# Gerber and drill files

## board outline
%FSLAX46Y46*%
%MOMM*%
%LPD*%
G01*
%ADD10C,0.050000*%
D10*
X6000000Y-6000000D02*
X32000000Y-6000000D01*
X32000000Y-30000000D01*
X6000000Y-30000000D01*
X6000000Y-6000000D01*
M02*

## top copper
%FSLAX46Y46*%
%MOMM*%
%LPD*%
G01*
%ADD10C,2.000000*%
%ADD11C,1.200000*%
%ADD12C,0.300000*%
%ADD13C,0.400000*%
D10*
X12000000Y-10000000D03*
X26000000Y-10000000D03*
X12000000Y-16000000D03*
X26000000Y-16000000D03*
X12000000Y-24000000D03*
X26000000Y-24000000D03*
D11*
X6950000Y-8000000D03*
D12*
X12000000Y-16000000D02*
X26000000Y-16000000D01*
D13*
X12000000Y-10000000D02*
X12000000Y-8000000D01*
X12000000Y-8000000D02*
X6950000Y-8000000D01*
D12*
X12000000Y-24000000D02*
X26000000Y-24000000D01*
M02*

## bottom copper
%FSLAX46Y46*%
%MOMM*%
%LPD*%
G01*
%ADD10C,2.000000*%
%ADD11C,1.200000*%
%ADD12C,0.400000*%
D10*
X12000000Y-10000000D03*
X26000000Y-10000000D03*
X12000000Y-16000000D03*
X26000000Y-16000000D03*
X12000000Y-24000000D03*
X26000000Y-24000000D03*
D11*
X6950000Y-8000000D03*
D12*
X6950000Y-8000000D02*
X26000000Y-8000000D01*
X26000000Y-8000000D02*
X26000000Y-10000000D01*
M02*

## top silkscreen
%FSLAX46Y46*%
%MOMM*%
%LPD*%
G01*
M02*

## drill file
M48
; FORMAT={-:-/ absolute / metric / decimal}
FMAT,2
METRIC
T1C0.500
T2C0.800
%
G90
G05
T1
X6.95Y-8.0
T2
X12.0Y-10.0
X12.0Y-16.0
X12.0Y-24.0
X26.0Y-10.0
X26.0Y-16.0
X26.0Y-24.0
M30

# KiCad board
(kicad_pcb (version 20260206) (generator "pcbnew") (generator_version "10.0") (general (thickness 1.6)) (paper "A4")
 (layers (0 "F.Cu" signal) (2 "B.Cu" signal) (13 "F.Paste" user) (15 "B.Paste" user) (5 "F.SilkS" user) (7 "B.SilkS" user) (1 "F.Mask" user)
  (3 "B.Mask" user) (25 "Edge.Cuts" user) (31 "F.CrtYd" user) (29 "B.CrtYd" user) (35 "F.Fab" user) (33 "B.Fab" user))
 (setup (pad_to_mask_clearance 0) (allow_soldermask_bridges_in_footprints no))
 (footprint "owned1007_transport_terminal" (layer "F.Cu") (at 12 10)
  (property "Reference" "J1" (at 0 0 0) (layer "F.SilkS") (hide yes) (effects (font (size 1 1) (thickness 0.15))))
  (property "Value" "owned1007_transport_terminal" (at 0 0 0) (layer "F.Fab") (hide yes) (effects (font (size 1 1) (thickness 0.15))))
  (pad "1" thru_hole circle (at 0 0) (size 2 2) (drill 0.8) (layers "*.Cu" "*.Mask") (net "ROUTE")))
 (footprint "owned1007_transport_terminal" (layer "F.Cu") (at 26 10)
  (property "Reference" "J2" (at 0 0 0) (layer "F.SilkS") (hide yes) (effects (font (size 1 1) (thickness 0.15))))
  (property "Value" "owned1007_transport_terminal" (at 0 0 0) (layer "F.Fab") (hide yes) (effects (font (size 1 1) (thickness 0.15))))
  (pad "1" thru_hole circle (at 0 0) (size 2 2) (drill 0.8) (layers "*.Cu" "*.Mask") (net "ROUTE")))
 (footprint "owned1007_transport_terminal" (layer "F.Cu") (at 12 16)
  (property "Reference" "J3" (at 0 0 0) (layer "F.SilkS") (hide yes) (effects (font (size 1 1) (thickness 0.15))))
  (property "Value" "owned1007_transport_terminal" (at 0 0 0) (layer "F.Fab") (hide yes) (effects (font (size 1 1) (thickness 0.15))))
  (pad "1" thru_hole circle (at 0 0) (size 2 2) (drill 0.8) (layers "*.Cu" "*.Mask") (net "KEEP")))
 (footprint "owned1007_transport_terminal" (layer "F.Cu") (at 26 16)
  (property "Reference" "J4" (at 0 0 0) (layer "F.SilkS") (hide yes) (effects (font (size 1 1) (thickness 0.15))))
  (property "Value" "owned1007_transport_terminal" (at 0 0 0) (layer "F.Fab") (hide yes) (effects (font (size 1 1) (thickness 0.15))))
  (pad "1" thru_hole circle (at 0 0) (size 2 2) (drill 0.8) (layers "*.Cu" "*.Mask") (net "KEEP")))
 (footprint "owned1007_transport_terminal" (layer "F.Cu") (at 12 24)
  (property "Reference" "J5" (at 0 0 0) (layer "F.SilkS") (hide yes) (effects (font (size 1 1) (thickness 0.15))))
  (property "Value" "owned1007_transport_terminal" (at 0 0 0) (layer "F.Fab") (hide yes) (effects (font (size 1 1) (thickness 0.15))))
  (pad "1" thru_hole circle (at 0 0) (size 2 2) (drill 0.8) (layers "*.Cu" "*.Mask") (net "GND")))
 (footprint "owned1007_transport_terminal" (layer "F.Cu") (at 26 24)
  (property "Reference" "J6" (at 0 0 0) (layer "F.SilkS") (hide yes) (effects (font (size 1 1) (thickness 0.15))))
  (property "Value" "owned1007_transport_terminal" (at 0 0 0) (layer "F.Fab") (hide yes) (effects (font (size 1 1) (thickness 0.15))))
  (pad "1" thru_hole circle (at 0 0) (size 2 2) (drill 0.8) (layers "*.Cu" "*.Mask") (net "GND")))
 (gr_rect (start 6 6) (end 32 30) (stroke (width 0.05) (type default)) (fill none) (layer "Edge.Cuts"))
 (segment (start 12 16) (end 26 16) (width 0.3) (layer "F.Cu") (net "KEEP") (locked yes))
 (segment (start 12 10) (end 12 8) (width 0.4) (layer "F.Cu") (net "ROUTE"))
 (segment (start 12 8) (end 6.95 8) (width 0.4) (layer "F.Cu") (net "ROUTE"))
 (segment (start 6.95 8) (end 26 8) (width 0.4) (layer "B.Cu") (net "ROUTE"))
 (segment (start 26 8) (end 26 10) (width 0.4) (layer "B.Cu") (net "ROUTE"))
 (via (at 6.95 8) (size 1.2) (drill 0.5) (layers "F.Cu" "B.Cu") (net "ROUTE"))
 (segment (start 12 24) (end 26 24) (width 0.3) (layer "F.Cu") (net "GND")))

